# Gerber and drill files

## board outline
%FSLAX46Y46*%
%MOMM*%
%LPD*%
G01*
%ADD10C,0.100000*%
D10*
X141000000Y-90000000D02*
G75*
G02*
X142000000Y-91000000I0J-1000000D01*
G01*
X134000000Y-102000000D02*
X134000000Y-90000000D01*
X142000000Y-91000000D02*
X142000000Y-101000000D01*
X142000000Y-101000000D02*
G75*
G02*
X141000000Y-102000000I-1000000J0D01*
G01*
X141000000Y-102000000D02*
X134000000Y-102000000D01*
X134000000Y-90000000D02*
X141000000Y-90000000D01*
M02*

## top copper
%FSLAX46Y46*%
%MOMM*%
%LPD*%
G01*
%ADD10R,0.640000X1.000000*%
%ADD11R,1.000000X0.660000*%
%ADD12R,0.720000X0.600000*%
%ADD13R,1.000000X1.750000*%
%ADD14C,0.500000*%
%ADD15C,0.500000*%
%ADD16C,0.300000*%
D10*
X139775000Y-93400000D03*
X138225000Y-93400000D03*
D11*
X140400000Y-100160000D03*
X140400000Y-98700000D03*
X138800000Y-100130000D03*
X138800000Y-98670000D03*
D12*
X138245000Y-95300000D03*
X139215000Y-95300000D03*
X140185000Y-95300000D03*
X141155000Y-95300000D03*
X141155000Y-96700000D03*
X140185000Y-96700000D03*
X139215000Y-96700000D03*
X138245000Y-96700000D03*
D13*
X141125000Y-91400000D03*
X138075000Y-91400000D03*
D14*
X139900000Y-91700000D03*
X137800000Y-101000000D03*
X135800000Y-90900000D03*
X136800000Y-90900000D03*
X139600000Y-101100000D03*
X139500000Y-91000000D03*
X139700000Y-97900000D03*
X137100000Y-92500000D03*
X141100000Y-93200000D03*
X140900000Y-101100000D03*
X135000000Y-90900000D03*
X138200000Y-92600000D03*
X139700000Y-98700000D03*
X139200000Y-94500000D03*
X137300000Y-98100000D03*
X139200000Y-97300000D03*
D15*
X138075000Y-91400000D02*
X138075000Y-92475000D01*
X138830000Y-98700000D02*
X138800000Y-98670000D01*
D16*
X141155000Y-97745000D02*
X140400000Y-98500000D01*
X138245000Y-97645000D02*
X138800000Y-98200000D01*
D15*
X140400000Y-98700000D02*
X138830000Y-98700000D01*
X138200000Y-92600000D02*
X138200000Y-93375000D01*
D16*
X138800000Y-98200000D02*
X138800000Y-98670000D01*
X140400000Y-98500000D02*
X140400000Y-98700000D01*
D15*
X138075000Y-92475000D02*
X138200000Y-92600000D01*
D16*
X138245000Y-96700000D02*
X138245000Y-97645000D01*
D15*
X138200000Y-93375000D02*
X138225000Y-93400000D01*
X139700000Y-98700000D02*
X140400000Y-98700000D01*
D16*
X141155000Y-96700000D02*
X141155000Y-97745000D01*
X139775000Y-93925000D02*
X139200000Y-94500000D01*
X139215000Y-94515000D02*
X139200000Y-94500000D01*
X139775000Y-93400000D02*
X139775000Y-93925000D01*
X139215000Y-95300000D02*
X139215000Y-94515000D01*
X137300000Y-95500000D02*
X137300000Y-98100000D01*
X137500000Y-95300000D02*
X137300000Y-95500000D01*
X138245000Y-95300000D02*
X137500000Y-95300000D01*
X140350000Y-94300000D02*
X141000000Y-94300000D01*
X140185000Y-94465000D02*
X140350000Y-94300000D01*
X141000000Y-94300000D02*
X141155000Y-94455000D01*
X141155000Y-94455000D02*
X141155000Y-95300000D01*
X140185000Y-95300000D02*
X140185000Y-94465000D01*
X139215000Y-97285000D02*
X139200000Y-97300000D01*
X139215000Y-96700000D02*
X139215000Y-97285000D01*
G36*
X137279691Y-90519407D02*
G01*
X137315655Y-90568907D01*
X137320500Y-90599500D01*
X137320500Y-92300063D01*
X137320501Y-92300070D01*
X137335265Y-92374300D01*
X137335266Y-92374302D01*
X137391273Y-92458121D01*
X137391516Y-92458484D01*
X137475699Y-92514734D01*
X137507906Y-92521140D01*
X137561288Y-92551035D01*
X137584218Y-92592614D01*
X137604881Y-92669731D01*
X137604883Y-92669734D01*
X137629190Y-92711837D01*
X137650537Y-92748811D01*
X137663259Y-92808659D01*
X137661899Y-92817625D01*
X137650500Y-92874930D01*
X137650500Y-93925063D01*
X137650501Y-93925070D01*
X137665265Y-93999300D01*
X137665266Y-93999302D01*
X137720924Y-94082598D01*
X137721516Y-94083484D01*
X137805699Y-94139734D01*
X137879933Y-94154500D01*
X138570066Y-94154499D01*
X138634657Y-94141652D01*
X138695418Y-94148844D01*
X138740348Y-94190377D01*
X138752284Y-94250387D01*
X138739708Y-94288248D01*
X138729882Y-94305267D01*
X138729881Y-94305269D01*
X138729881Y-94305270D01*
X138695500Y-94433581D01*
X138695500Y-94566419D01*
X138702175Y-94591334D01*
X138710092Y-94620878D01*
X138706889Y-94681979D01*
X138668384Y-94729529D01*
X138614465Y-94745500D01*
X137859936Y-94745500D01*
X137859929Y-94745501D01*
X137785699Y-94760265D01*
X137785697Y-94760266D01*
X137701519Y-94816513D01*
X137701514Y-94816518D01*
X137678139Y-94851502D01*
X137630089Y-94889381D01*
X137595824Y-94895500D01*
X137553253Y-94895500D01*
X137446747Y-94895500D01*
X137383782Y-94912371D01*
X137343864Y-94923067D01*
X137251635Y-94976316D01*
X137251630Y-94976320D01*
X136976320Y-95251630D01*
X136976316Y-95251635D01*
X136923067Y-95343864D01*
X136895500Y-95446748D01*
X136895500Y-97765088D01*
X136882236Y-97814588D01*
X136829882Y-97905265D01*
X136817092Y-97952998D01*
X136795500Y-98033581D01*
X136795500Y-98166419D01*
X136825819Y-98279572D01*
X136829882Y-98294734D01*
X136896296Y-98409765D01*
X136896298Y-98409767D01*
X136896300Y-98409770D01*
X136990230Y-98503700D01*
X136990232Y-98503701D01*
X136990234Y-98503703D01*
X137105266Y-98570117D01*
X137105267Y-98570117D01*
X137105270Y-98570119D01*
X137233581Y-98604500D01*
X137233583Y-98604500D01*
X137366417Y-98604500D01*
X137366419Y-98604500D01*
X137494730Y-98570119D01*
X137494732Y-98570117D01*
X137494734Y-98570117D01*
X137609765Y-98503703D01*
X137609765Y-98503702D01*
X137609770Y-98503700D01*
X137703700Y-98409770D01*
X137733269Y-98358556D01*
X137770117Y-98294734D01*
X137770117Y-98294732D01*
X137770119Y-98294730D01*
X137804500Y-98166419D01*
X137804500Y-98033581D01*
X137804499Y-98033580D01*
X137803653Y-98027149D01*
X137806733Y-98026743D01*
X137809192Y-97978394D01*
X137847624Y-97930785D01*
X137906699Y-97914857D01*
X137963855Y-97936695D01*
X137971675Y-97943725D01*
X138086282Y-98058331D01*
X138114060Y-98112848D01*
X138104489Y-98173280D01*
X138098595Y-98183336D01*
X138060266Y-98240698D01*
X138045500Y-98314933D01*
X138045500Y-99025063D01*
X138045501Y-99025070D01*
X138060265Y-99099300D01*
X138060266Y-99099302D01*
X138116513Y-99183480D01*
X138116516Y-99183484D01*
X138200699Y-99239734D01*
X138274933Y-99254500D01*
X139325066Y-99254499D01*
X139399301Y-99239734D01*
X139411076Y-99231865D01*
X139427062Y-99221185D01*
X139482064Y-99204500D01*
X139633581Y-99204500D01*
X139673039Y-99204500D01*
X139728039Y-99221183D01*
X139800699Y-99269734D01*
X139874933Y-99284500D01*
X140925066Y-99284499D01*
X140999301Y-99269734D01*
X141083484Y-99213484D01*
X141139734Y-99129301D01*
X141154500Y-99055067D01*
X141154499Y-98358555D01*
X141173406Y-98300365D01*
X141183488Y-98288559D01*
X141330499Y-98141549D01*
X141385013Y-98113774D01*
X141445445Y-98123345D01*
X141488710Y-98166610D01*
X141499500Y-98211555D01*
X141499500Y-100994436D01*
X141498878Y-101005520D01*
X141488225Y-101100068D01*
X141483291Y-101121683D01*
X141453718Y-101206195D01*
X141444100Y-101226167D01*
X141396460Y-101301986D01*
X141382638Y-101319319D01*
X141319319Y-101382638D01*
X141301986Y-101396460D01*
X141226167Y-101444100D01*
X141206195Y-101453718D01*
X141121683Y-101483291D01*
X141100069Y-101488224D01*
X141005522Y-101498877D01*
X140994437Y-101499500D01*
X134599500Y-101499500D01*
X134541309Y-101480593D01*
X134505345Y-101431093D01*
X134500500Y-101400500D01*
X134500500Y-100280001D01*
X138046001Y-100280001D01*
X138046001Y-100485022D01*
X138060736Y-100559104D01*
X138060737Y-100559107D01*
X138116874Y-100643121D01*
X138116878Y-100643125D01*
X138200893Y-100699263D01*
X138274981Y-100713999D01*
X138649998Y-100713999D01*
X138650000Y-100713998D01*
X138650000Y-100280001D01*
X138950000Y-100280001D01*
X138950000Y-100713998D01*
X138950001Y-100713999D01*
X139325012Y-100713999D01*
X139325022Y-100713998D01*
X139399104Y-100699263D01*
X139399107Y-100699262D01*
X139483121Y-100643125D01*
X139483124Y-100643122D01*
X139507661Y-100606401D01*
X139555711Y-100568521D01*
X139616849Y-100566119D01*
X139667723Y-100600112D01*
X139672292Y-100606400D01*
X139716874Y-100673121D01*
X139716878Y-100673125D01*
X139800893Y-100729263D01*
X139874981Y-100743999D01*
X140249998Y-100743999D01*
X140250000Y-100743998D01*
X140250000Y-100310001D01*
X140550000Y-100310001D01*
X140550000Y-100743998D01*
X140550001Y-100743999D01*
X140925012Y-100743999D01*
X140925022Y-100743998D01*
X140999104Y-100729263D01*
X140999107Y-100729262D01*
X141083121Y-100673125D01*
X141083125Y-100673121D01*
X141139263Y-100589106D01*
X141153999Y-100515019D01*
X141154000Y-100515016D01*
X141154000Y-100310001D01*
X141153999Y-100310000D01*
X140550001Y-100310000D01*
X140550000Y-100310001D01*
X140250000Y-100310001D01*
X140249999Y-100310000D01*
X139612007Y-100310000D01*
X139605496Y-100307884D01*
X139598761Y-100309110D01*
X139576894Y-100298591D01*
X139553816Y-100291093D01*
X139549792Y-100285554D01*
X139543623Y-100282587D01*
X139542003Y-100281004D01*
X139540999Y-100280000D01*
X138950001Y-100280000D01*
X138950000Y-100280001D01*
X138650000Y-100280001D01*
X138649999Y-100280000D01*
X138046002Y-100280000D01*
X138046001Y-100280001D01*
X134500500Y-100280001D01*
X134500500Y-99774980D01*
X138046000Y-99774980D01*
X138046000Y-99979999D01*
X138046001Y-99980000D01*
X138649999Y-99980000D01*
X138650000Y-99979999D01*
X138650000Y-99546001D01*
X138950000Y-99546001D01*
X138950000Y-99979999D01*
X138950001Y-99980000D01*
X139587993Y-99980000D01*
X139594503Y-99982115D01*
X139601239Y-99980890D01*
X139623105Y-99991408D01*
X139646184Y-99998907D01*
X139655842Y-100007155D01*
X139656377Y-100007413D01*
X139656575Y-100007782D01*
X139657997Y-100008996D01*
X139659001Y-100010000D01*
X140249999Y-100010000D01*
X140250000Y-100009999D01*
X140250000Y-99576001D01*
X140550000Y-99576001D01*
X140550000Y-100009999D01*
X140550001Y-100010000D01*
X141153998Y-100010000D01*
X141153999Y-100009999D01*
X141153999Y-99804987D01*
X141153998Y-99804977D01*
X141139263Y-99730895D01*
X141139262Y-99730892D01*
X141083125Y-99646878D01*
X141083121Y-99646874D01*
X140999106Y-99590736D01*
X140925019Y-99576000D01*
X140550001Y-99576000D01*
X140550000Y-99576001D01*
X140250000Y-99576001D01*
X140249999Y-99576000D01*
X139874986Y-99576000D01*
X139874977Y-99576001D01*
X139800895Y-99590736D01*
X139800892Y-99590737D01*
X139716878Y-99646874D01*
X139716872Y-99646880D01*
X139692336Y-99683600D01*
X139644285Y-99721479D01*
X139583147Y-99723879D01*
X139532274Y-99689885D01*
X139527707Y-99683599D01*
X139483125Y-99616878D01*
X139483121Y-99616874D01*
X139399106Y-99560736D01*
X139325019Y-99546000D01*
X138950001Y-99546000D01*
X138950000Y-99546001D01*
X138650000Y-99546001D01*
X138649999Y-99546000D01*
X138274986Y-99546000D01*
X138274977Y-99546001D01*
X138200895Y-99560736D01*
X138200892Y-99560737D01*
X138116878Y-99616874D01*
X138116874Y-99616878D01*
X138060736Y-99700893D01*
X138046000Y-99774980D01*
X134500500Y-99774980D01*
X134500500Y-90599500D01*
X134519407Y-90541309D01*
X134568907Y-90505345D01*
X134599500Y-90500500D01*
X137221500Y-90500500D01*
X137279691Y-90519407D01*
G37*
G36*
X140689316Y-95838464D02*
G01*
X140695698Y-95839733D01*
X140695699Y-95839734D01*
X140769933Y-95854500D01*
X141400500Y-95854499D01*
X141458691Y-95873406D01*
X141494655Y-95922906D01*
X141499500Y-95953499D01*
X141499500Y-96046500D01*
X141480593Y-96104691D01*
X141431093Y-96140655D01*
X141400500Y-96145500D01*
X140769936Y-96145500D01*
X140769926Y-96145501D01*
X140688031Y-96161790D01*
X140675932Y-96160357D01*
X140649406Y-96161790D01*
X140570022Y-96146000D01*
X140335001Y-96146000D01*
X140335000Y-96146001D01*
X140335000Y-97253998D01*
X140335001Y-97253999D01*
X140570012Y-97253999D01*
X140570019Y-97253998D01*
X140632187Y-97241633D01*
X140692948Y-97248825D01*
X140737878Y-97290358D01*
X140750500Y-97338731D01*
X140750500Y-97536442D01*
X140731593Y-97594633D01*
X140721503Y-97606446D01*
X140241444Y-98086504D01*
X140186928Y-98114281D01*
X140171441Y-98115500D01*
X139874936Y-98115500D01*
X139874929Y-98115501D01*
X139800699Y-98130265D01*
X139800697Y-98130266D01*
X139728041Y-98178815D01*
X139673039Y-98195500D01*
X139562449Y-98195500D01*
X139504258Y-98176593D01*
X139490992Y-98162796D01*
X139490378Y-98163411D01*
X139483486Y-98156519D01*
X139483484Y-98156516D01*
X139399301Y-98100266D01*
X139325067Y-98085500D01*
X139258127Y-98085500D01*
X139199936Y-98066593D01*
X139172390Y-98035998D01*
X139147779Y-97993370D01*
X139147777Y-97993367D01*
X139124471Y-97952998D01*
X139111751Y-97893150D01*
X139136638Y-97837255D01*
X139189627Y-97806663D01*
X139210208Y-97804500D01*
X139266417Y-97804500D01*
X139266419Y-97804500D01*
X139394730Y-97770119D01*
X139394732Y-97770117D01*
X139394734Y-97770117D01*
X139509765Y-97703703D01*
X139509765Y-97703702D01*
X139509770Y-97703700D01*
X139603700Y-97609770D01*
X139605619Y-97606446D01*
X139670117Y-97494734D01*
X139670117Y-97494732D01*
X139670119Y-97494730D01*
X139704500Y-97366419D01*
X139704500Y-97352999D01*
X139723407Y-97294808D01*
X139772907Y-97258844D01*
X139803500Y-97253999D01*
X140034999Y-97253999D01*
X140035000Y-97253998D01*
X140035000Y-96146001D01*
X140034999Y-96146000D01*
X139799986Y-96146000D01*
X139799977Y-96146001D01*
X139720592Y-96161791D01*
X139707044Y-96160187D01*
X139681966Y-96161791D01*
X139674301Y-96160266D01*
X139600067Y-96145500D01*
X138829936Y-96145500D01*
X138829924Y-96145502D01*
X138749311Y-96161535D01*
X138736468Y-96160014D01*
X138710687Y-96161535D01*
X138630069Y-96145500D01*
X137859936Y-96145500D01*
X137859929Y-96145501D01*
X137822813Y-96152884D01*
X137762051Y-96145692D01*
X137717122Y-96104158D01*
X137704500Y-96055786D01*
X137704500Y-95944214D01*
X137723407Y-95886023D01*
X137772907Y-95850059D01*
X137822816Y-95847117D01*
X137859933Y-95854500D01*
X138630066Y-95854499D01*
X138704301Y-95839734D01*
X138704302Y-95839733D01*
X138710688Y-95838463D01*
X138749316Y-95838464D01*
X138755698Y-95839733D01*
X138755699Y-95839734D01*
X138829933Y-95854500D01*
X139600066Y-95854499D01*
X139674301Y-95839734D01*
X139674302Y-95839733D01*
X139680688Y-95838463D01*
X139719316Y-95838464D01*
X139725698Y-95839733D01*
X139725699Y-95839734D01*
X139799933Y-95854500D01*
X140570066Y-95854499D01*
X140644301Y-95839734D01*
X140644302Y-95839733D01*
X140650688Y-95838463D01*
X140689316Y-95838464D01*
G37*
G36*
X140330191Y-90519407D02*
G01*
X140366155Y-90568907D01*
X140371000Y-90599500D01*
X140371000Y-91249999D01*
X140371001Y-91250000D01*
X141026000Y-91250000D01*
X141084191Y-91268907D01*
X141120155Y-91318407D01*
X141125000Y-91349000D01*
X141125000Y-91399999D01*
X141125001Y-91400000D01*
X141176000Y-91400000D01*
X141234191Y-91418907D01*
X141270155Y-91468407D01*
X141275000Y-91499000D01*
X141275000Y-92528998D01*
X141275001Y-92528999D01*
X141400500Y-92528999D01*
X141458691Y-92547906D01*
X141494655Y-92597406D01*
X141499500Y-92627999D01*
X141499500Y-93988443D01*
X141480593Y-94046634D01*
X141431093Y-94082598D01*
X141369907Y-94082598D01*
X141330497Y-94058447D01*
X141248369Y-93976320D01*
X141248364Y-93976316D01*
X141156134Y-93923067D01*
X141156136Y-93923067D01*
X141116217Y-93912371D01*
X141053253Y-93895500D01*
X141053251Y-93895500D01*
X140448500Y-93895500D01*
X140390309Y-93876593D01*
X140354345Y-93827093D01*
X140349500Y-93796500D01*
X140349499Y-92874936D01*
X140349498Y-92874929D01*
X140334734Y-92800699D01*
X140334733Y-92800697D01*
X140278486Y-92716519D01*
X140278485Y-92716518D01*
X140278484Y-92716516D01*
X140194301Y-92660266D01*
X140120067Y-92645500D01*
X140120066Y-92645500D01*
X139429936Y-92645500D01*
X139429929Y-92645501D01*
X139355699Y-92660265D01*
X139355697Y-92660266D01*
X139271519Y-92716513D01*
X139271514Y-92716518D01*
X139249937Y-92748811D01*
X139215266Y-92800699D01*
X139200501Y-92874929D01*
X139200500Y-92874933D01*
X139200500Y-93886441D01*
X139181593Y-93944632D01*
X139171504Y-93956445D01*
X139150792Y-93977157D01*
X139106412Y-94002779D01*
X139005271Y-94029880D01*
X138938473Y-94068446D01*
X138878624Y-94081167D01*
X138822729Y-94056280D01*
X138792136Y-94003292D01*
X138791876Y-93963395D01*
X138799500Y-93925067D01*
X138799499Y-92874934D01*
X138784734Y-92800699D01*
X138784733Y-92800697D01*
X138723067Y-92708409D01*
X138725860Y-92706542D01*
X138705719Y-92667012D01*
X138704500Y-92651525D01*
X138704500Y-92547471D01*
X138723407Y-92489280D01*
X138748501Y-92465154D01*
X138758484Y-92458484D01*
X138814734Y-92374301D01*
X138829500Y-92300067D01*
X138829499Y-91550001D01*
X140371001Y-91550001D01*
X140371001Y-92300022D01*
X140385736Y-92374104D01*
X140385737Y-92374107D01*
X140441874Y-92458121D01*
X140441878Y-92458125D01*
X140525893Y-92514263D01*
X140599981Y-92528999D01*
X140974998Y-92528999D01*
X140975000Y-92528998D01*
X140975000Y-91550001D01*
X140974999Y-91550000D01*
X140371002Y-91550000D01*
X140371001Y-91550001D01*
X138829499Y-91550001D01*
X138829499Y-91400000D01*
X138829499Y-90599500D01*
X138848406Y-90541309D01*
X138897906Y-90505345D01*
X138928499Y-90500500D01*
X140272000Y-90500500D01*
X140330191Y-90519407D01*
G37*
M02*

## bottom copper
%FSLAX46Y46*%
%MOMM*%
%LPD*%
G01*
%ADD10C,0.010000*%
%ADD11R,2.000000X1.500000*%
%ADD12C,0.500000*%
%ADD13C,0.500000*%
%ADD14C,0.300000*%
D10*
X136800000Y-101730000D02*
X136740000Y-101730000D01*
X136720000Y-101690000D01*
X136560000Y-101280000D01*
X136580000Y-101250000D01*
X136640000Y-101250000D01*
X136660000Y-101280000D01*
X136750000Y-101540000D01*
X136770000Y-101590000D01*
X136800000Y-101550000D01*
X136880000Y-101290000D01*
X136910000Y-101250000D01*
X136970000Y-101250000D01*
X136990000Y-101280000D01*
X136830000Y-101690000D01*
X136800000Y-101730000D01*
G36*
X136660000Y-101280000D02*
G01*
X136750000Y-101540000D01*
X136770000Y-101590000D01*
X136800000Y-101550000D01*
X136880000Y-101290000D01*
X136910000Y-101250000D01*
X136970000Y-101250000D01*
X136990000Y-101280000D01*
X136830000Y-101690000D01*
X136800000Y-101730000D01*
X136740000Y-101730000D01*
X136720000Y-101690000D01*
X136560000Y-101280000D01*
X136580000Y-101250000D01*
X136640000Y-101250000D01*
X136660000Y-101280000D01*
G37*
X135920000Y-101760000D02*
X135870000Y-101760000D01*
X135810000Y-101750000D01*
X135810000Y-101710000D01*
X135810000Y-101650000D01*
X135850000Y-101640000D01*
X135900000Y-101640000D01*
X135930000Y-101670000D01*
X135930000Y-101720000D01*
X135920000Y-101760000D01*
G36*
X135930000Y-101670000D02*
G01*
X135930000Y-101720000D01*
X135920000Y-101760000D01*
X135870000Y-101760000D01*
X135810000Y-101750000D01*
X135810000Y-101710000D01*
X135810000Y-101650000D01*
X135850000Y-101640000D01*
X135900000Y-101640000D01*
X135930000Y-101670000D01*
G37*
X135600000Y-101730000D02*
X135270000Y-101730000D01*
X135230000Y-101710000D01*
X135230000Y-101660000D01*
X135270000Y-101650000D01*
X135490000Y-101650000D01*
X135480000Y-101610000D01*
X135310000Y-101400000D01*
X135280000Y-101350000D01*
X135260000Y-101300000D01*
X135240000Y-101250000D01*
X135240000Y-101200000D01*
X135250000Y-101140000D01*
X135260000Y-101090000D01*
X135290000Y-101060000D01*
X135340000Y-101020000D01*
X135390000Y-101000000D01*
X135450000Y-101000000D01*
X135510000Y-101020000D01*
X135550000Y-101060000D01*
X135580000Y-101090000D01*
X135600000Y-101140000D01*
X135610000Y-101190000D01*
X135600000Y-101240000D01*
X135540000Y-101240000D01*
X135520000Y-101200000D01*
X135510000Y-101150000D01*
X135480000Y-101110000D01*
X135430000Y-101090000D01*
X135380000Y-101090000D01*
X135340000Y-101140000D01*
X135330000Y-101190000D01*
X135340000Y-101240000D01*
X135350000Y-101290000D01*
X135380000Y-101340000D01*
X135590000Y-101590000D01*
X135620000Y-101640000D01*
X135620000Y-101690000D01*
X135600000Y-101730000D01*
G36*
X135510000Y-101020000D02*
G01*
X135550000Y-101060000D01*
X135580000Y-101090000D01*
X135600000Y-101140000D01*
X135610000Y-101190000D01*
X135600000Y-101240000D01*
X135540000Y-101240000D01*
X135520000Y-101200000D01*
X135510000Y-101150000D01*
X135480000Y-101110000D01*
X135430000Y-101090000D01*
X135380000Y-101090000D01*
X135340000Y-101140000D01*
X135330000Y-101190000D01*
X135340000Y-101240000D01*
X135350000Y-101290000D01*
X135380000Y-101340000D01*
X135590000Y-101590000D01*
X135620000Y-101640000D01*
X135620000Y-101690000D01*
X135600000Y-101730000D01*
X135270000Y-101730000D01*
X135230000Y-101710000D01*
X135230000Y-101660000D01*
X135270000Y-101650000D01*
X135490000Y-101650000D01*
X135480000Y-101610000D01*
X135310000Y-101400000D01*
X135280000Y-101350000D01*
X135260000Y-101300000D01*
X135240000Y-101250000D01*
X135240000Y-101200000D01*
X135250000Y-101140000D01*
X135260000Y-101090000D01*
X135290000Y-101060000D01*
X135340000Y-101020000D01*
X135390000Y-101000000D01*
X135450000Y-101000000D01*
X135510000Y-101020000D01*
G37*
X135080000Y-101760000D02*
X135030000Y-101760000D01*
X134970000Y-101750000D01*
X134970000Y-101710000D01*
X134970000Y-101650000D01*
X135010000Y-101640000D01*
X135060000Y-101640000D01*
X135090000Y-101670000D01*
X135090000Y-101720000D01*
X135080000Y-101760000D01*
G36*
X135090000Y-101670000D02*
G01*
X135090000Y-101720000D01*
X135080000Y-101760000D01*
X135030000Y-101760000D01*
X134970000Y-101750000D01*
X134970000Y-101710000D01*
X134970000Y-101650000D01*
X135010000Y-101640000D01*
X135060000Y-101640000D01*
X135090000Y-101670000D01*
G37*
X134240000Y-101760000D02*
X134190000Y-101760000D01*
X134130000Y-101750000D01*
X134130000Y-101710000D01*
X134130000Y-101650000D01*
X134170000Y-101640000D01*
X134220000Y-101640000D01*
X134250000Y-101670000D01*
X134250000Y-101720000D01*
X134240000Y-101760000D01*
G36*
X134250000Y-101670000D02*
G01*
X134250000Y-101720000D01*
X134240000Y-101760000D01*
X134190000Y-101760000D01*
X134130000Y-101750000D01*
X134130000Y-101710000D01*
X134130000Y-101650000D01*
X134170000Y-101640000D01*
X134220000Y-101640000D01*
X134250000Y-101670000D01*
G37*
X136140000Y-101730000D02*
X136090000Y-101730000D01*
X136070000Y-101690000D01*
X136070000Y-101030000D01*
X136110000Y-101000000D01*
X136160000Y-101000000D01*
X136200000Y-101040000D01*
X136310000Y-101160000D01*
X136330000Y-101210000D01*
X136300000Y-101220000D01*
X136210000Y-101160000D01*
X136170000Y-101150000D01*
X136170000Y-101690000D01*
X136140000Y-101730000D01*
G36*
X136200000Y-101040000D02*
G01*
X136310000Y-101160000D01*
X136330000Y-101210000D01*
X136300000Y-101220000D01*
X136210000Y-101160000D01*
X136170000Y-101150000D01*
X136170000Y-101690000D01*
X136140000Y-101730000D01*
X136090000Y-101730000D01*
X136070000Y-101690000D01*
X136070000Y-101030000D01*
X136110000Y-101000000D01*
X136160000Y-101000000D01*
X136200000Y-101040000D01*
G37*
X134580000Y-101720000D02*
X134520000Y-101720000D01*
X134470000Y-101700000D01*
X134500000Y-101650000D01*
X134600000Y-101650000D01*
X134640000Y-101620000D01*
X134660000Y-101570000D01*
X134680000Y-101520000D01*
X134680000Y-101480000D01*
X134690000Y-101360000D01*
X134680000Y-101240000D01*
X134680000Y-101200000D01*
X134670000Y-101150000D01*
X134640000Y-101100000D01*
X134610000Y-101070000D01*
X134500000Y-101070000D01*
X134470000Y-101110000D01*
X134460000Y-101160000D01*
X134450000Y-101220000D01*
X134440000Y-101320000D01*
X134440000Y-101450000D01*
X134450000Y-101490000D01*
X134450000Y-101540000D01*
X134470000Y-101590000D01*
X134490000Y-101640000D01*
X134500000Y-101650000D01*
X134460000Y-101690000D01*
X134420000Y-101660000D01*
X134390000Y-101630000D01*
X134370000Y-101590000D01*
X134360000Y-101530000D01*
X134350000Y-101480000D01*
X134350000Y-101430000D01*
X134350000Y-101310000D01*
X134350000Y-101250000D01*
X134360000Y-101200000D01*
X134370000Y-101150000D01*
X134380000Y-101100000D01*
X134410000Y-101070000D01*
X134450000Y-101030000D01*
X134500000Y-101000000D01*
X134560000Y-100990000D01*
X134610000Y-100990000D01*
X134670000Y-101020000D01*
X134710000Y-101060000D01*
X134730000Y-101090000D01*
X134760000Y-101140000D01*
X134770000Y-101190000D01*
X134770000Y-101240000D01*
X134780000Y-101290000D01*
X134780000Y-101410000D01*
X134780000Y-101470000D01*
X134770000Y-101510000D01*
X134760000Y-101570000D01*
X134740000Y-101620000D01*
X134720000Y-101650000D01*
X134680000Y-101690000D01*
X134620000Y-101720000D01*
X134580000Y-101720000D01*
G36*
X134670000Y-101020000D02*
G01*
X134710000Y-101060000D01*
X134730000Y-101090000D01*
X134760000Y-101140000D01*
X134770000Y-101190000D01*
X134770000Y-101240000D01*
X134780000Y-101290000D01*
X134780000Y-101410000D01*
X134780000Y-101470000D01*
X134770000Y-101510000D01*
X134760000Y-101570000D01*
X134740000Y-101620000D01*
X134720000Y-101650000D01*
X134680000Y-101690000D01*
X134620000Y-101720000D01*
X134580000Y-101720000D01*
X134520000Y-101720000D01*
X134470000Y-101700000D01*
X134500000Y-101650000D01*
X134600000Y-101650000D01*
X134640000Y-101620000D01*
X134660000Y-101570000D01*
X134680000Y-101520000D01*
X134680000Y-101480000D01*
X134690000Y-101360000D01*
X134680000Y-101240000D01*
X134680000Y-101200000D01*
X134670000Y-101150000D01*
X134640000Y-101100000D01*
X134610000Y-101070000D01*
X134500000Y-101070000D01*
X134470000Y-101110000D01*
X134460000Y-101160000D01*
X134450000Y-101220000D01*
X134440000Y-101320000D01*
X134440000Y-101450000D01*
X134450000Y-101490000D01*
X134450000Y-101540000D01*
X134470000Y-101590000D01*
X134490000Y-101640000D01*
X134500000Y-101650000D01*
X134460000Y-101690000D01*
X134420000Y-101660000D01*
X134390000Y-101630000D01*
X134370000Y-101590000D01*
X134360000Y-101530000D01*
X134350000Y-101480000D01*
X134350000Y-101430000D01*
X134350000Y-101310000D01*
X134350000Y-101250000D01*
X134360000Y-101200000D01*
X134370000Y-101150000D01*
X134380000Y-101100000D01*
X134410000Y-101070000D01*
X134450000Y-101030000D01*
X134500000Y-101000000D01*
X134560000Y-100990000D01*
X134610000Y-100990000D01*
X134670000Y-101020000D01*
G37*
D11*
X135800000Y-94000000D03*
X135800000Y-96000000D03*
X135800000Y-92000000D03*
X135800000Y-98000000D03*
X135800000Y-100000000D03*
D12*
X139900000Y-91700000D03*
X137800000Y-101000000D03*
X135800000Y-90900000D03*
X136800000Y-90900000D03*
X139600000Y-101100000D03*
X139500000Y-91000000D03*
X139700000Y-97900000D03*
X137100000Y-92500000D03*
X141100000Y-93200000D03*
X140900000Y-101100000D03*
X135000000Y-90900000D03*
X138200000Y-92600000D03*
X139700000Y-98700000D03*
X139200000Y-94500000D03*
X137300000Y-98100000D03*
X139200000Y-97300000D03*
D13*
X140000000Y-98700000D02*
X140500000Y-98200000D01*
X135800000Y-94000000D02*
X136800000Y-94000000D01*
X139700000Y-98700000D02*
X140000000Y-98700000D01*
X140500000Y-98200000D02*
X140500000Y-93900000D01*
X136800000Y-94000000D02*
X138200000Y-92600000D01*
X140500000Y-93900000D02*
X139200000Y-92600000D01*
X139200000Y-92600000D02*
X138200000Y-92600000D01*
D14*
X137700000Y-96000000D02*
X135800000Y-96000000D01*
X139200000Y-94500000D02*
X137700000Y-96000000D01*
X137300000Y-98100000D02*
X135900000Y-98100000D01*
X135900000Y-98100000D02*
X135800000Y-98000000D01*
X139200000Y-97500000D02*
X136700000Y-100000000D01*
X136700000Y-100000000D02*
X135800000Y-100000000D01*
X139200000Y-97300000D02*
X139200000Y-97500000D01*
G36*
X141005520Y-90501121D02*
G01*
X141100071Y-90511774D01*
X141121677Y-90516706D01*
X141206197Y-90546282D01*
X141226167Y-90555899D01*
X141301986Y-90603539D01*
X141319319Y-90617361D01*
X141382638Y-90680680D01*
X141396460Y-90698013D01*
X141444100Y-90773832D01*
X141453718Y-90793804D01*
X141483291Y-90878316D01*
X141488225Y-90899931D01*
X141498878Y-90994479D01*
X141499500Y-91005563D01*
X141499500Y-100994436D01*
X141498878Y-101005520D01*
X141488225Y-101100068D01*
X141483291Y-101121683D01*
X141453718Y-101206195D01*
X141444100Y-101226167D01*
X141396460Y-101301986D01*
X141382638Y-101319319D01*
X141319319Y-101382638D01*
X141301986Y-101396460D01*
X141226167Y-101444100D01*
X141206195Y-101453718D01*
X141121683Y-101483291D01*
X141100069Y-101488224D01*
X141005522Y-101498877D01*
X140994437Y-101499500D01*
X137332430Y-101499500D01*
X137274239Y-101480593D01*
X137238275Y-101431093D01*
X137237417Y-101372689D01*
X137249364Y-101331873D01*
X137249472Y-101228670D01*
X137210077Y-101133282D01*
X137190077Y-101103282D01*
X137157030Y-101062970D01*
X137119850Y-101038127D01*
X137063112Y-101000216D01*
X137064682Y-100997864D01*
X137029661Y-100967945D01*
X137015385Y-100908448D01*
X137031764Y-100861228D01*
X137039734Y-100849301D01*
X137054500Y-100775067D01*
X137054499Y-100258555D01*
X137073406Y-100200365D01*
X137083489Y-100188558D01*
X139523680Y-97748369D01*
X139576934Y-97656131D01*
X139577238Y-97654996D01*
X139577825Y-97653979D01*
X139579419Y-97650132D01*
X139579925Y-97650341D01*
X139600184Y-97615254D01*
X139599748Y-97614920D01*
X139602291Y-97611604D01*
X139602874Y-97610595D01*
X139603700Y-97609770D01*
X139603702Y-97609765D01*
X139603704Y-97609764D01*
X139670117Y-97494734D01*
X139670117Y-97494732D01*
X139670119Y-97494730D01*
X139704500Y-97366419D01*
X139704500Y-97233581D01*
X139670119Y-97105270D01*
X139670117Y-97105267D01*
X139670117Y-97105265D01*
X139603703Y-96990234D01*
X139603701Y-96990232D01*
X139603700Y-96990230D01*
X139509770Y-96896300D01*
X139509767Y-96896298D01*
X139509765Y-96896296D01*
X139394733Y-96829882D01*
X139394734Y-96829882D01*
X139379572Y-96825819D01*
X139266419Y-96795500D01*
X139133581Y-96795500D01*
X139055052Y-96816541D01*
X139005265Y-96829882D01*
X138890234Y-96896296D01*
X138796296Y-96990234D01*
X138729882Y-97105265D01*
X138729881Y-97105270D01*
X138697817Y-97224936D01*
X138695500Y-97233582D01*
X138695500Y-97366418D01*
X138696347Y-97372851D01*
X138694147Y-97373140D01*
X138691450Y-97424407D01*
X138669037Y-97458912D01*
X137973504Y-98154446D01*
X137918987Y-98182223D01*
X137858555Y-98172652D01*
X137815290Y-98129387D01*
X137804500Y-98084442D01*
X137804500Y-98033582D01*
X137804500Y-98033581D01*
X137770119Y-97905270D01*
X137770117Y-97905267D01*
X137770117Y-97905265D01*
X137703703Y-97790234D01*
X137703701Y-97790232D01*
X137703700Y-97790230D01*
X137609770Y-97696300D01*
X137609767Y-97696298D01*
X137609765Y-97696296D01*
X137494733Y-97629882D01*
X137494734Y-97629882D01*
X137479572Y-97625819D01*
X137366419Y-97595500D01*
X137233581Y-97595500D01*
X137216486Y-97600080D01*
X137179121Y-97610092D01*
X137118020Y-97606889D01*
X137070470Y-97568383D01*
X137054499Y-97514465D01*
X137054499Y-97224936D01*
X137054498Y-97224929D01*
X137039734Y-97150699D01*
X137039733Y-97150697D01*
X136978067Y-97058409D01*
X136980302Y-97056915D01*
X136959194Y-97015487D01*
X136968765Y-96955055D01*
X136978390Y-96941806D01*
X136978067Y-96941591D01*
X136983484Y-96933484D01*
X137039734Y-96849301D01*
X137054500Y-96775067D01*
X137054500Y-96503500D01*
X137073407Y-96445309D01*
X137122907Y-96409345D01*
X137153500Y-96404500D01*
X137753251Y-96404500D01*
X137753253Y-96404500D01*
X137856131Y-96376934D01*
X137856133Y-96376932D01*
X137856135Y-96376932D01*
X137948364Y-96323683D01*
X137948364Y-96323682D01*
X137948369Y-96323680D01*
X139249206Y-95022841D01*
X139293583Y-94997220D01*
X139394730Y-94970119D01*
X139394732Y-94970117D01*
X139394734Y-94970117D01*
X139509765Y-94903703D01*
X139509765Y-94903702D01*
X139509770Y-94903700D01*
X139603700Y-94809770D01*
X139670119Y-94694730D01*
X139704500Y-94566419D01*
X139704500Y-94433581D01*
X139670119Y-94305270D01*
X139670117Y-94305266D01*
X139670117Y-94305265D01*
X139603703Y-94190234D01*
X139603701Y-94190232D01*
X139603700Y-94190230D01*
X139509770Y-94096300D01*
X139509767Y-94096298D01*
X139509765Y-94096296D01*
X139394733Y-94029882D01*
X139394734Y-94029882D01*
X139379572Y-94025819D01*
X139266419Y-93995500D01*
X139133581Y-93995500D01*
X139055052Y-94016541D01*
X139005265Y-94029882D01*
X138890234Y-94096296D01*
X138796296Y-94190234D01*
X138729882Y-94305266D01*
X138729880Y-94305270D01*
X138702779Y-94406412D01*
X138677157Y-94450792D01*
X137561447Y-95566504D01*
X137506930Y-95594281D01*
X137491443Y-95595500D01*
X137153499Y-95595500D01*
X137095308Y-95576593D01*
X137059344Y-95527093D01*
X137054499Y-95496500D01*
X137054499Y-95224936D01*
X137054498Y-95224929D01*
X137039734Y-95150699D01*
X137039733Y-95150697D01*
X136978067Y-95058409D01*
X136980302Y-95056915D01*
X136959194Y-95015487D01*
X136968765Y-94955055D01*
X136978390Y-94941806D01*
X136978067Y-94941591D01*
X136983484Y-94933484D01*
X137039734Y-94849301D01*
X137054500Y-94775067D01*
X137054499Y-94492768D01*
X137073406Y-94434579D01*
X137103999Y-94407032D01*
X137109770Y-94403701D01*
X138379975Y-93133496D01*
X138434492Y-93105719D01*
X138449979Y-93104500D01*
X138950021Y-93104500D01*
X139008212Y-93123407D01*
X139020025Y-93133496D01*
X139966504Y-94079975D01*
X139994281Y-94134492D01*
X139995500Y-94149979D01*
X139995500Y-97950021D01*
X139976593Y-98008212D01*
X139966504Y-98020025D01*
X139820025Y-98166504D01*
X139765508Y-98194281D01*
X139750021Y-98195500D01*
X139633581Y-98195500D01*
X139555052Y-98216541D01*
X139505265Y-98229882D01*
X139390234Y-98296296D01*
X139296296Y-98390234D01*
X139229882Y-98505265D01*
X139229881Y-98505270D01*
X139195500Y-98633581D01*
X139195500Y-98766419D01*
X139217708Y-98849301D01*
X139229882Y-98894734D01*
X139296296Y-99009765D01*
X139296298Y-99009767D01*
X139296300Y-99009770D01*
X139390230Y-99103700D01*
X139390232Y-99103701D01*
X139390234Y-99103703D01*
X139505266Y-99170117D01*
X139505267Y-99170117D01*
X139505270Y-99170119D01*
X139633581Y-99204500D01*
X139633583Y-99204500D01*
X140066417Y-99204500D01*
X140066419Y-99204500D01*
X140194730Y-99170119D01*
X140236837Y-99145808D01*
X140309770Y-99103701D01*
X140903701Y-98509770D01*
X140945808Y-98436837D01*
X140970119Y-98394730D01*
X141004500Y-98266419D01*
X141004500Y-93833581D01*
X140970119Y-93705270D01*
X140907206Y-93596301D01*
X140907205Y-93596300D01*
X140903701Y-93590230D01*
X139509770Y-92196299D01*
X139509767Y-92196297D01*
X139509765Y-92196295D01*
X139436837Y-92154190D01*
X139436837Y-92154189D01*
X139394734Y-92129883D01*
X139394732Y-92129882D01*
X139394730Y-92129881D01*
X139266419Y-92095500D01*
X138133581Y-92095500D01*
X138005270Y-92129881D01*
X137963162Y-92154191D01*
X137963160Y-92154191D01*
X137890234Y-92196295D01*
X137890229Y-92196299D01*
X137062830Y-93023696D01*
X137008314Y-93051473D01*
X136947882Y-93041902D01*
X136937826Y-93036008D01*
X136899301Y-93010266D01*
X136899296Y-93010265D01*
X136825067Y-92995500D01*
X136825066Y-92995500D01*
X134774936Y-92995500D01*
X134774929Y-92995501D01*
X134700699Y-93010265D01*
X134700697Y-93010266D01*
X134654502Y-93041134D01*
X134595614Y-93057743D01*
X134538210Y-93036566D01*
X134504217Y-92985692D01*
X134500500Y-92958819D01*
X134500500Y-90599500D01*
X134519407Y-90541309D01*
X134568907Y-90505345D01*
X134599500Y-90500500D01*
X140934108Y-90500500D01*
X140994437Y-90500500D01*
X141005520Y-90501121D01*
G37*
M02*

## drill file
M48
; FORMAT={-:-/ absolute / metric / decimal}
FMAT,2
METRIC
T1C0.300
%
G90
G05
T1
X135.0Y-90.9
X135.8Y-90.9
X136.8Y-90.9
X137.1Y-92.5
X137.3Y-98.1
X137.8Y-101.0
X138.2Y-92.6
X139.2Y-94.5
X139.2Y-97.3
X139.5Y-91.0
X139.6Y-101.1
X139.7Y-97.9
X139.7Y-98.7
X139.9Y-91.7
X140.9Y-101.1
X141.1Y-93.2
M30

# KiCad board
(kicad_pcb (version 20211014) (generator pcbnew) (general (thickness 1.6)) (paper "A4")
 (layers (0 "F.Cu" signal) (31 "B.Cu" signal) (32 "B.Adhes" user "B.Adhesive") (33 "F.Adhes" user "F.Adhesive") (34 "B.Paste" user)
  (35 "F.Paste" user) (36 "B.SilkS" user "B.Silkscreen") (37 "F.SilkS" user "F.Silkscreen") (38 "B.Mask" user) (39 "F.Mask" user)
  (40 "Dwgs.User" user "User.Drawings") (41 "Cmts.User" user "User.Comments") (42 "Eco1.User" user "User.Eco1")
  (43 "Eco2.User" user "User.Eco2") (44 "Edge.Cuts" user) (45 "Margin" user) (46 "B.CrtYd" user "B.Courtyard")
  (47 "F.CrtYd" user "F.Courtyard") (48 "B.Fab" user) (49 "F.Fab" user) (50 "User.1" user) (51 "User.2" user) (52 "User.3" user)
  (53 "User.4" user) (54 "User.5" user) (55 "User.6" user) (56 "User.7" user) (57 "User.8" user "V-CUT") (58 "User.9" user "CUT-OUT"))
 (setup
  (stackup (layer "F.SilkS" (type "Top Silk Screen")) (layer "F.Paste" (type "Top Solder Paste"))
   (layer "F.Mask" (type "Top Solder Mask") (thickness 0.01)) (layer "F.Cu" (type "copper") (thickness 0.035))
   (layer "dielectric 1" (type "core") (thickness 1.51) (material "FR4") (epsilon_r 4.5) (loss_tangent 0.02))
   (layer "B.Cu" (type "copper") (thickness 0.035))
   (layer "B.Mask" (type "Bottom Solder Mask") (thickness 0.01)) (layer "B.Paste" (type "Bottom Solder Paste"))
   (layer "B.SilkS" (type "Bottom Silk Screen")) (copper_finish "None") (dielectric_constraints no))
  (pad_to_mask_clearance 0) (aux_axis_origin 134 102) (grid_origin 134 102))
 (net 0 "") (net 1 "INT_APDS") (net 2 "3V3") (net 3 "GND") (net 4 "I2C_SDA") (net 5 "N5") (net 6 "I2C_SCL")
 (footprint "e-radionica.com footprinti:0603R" (layer "F.Cu") (at 139 93.4 180)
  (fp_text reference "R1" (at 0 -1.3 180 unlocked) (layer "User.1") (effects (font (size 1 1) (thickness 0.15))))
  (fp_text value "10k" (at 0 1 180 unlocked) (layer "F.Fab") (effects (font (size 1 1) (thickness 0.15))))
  (pad "1" smd rect locked (at -0.775 0 270) (size 1 0.64) (layers "F.Cu" "F.Paste" "F.Mask") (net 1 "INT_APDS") (solder_mask_margin 0.1))
  (pad "2" smd rect locked (at 0.775 0 270) (size 1 0.64) (layers "F.Cu" "F.Paste" "F.Mask") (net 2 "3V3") (solder_mask_margin 0.1)))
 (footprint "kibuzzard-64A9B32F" (layer "F.Cu") (at 135 96 -90)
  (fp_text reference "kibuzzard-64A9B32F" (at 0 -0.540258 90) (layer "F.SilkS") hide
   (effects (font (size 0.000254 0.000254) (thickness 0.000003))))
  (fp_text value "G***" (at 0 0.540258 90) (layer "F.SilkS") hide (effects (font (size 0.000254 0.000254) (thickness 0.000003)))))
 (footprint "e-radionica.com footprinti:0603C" (layer "F.Cu") (at 140.4 99.43 90)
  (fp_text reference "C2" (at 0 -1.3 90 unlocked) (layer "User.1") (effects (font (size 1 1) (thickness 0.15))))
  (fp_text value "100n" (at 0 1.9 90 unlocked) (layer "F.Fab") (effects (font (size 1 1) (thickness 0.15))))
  (pad "1" smd rect locked (at -0.73 0 90) (size 0.66 1) (layers "F.Cu" "F.Paste" "F.Mask") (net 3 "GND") (solder_mask_margin 0.1))
  (pad "2" smd rect locked (at 0.73 0 90) (size 0.66 1) (layers "F.Cu" "F.Paste" "F.Mask") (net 2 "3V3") (solder_mask_margin 0.1)))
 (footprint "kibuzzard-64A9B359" (layer "F.Cu") (at 136.5 96 -90)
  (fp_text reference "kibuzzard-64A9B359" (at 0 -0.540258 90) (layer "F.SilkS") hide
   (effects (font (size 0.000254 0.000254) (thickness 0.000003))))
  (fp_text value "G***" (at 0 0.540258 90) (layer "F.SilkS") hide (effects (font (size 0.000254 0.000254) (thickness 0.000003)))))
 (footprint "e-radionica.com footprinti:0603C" (layer "F.Cu") (at 138.8 99.4 90)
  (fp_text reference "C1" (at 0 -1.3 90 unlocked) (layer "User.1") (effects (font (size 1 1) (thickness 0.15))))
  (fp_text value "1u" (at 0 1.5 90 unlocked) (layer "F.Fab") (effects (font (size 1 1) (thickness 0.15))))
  (pad "1" smd rect locked (at -0.73 0 90) (size 0.66 1) (layers "F.Cu" "F.Paste" "F.Mask") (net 3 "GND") (solder_mask_margin 0.1))
  (pad "2" smd rect locked (at 0.73 0 90) (size 0.66 1) (layers "F.Cu" "F.Paste" "F.Mask") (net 2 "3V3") (solder_mask_margin 0.1)))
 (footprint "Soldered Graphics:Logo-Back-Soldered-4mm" (layer "F.Cu") (at 139.5 96 90)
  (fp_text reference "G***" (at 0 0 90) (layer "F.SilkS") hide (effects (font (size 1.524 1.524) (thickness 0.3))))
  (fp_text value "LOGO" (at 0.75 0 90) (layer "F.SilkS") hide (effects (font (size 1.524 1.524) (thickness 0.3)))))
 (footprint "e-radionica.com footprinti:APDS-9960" (layer "F.Cu") (at 139.7 96 90)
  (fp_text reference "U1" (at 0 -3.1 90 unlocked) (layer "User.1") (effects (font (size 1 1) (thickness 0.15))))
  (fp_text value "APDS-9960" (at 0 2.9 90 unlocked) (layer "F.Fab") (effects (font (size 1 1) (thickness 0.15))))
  (pad "1" smd rect (at 0.7 -1.455 90) (size 0.6 0.72) (layers "F.Cu" "F.Paste" "F.Mask") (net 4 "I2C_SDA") (solder_mask_margin 0.1))
  (pad "2" smd rect (at 0.7 -0.485 90) (size 0.6 0.72) (layers "F.Cu" "F.Paste" "F.Mask") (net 1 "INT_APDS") (solder_mask_margin 0.1))
  (pad "3" smd rect (at 0.7 0.485 90) (size 0.6 0.72) (layers "F.Cu" "F.Paste" "F.Mask") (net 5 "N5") (solder_mask_margin 0.1))
  (pad "4" smd rect (at 0.7 1.455 90) (size 0.6 0.72) (layers "F.Cu" "F.Paste" "F.Mask") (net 5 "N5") (solder_mask_margin 0.1))
  (pad "5" smd rect (at -0.7 1.455 90) (size 0.6 0.72) (layers "F.Cu" "F.Paste" "F.Mask") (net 2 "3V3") (solder_mask_margin 0.1))
  (pad "6" smd rect (at -0.7 0.485 90) (size 0.6 0.72) (layers "F.Cu" "F.Paste" "F.Mask") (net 3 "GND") (solder_mask_margin 0.1))
  (pad "7" smd rect (at -0.7 -0.485 90) (size 0.6 0.72) (layers "F.Cu" "F.Paste" "F.Mask") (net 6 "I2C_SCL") (solder_mask_margin 0.1))
  (pad "8" smd rect (at -0.7 -1.455 90) (size 0.6 0.72) (layers "F.Cu" "F.Paste" "F.Mask") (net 2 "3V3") (solder_mask_margin 0.1)))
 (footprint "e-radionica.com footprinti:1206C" (layer "F.Cu") (at 139.6 91.4 180)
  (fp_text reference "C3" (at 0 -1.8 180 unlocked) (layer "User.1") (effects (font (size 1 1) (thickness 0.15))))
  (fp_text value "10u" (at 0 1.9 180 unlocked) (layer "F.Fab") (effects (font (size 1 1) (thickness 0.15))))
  (pad "1" smd rect locked (at -1.525 0 270) (size 1.75 1) (layers "F.Cu" "F.Paste" "F.Mask") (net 3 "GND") (solder_mask_margin 0.1))
  (pad "2" smd rect locked (at 1.525 0 270) (size 1.75 1) (layers "F.Cu" "F.Paste" "F.Mask") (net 2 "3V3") (solder_mask_margin 0.1)))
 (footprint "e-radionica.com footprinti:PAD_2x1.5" (layer "B.Cu") (at 135.8 94 180)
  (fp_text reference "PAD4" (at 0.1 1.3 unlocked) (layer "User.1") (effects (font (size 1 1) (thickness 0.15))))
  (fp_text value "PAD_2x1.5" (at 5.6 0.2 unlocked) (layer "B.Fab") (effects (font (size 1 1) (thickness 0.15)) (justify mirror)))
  (pad "1" smd rect (at 0 0 180) (size 2 1.5) (layers "B.Cu" "B.Paste" "B.Mask") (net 2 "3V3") (solder_mask_margin 0.1)))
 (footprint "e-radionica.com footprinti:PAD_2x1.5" (layer "B.Cu") (at 135.8 96 180)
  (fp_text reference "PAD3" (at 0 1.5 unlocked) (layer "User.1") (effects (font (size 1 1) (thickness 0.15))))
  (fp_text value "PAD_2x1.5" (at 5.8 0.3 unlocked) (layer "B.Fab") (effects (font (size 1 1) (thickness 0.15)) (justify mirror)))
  (pad "1" smd rect (at 0 0 180) (size 2 1.5) (layers "B.Cu" "B.Paste" "B.Mask") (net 1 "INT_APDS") (solder_mask_margin 0.1)))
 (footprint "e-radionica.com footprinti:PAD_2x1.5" (layer "B.Cu") (at 135.8 92 180)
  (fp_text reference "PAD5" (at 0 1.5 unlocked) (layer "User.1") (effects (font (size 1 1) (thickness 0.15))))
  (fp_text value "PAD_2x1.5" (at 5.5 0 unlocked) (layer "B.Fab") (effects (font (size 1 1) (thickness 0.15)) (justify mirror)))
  (pad "1" smd rect (at 0 0 180) (size 2 1.5) (layers "B.Cu" "B.Paste" "B.Mask") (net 3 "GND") (solder_mask_margin 0.1) (zone_connect 2)))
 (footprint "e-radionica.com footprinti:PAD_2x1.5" (layer "B.Cu") (at 135.8 98 180)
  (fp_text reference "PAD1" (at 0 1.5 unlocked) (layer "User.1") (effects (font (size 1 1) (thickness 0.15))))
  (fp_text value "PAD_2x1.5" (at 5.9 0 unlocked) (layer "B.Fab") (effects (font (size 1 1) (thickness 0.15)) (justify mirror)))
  (pad "1" smd rect (at 0 0 180) (size 2 1.5) (layers "B.Cu" "B.Paste" "B.Mask") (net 4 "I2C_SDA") (solder_mask_margin 0.1)))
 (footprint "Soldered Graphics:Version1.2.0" (layer "B.Cu") (at 135.5 101.4 180)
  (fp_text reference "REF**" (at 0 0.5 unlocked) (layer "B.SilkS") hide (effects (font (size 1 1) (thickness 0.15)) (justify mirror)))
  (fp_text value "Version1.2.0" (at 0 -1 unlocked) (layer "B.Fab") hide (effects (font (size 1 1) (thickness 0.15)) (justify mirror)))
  (fp_poly
   (pts (xy -1.3 -0.33) (xy -1.24 -0.33) (xy -1.22 -0.29) (xy -1.06 0.12) (xy -1.08 0.15) (xy -1.14 0.15) (xy -1.16 0.12) (xy -1.25 -0.14)
    (xy -1.27 -0.19) (xy -1.3 -0.15) (xy -1.38 0.11) (xy -1.41 0.15) (xy -1.47 0.15) (xy -1.49 0.12) (xy -1.33 -0.29) (xy -1.3 -0.33))
   (layer "B.Cu") (width 0.01) (fill solid))
  (fp_poly
   (pts (xy -0.42 -0.36) (xy -0.37 -0.36) (xy -0.31 -0.35) (xy -0.31 -0.31) (xy -0.31 -0.25) (xy -0.35 -0.24) (xy -0.4 -0.24)
    (xy -0.43 -0.27) (xy -0.43 -0.32) (xy -0.42 -0.36))
   (layer "B.Cu") (width 0.01) (fill solid))
  (fp_poly
   (pts (xy -0.1 -0.33) (xy 0.23 -0.33) (xy 0.27 -0.31) (xy 0.27 -0.26) (xy 0.23 -0.25) (xy 0.01 -0.25) (xy 0.02 -0.21) (xy 0.19 0)
    (xy 0.22 0.05) (xy 0.24 0.1) (xy 0.26 0.15) (xy 0.26 0.2) (xy 0.25 0.26) (xy 0.24 0.31) (xy 0.21 0.34) (xy 0.16 0.38) (xy 0.11 0.4)
    (xy 0.05 0.4) (xy -0.01 0.38) (xy -0.05 0.34) (xy -0.08 0.31) (xy -0.1 0.26) (xy -0.11 0.21) (xy -0.1 0.16) (xy -0.04 0.16)
    (xy -0.02 0.2) (xy -0.01 0.25) (xy 0.02 0.29) (xy 0.07 0.31) (xy 0.12 0.31) (xy 0.16 0.26) (xy 0.17 0.21) (xy 0.16 0.16) (xy 0.15 0.11)
    (xy 0.12 0.06) (xy -0.09 -0.19) (xy -0.12 -0.24) (xy -0.12 -0.29) (xy -0.1 -0.33))
   (layer "B.Cu") (width 0.01) (fill solid))
  (fp_poly
   (pts (xy 0.42 -0.36) (xy 0.47 -0.36) (xy 0.53 -0.35) (xy 0.53 -0.31) (xy 0.53 -0.25) (xy 0.49 -0.24) (xy 0.44 -0.24) (xy 0.41 -0.27)
    (xy 0.41 -0.32) (xy 0.42 -0.36))
   (layer "B.Cu") (width 0.01) (fill solid))
  (fp_poly
   (pts (xy 1.26 -0.36) (xy 1.31 -0.36) (xy 1.37 -0.35) (xy 1.37 -0.31) (xy 1.37 -0.25) (xy 1.33 -0.24) (xy 1.28 -0.24) (xy 1.25 -0.27)
    (xy 1.25 -0.32) (xy 1.26 -0.36))
   (layer "B.Cu") (width 0.01) (fill solid))
  (fp_poly
   (pts (xy -0.64 -0.33) (xy -0.59 -0.33) (xy -0.57 -0.29) (xy -0.57 0.37) (xy -0.61 0.4) (xy -0.66 0.4) (xy -0.7 0.36) (xy -0.81 0.24)
    (xy -0.83 0.19) (xy -0.8 0.18) (xy -0.71 0.24) (xy -0.67 0.25) (xy -0.67 -0.29) (xy -0.64 -0.33))
   (layer "B.Cu") (width 0.01) (fill solid))
  (fp_poly
   (pts (xy 0.92 -0.32) (xy 0.98 -0.32) (xy 1.03 -0.3) (xy 1 -0.25) (xy 0.9 -0.25) (xy 0.86 -0.22) (xy 0.84 -0.17) (xy 0.82 -0.12)
    (xy 0.82 -0.08) (xy 0.81 0.04) (xy 0.82 0.16) (xy 0.82 0.2) (xy 0.83 0.25) (xy 0.86 0.3) (xy 0.89 0.33) (xy 1 0.33) (xy 1.03 0.29)
    (xy 1.04 0.24) (xy 1.05 0.18) (xy 1.06 0.08) (xy 1.06 -0.05) (xy 1.05 -0.09) (xy 1.05 -0.14) (xy 1.03 -0.19) (xy 1.01 -0.24)
    (xy 1 -0.25) (xy 1.04 -0.29) (xy 1.08 -0.26) (xy 1.11 -0.23) (xy 1.13 -0.19) (xy 1.14 -0.13) (xy 1.15 -0.08) (xy 1.15 -0.03)
    (xy 1.15 0.09) (xy 1.15 0.15) (xy 1.14 0.2) (xy 1.13 0.25) (xy 1.12 0.3) (xy 1.09 0.33) (xy 1.05 0.37) (xy 1 0.4) (xy 0.94 0.41)
    (xy 0.89 0.41) (xy 0.83 0.38) (xy 0.79 0.34) (xy 0.77 0.31) (xy 0.74 0.26) (xy 0.73 0.21) (xy 0.73 0.16) (xy 0.72 0.11) (xy 0.72 -0.01)
    (xy 0.72 -0.07) (xy 0.73 -0.11) (xy 0.74 -0.17) (xy 0.76 -0.22) (xy 0.78 -0.25) (xy 0.82 -0.29) (xy 0.88 -0.32) (xy 0.92 -0.32))
   (layer "B.Cu") (width 0.01) (fill solid)))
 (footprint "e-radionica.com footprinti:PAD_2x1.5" (layer "B.Cu") (at 135.8 100 180)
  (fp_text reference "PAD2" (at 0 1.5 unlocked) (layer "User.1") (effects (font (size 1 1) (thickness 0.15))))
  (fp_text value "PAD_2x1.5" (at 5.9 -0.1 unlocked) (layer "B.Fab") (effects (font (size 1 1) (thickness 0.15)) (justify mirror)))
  (pad "1" smd rect (at 0 0 180) (size 2 1.5) (layers "B.Cu" "B.Paste" "B.Mask") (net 6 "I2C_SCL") (solder_mask_margin 0.1)))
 (gr_arc (start 141 90) (mid 141.707107 90.292893) (end 142 91) (layer "Edge.Cuts") (width 0.1))
 (gr_line (start 134 102) (end 134 90) (layer "Edge.Cuts") (width 0.1))
 (gr_line (start 142 91) (end 142 101) (layer "Edge.Cuts") (width 0.1))
 (gr_arc (start 142 101) (mid 141.707107 101.707107) (end 141 102) (layer "Edge.Cuts") (width 0.1))
 (gr_line (start 141 102) (end 134 102) (layer "Edge.Cuts") (width 0.1))
 (gr_line (start 134 90) (end 141 90) (layer "Edge.Cuts") (width 0.1))
 (via (at 139.9 91.7) (size 0.5) (drill 0.3) (layers "F.Cu" "B.Cu") (free) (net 3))
 (via (at 137.8 101) (size 0.5) (drill 0.3) (layers "F.Cu" "B.Cu") (free) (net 3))
 (via (at 135.8 90.9) (size 0.5) (drill 0.3) (layers "F.Cu" "B.Cu") (free) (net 3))
 (via (at 136.8 90.9) (size 0.5) (drill 0.3) (layers "F.Cu" "B.Cu") (free) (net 3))
 (via (at 139.6 101.1) (size 0.5) (drill 0.3) (layers "F.Cu" "B.Cu") (free) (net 3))
 (via (at 139.5 91) (size 0.5) (drill 0.3) (layers "F.Cu" "B.Cu") (free) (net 3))
 (via (at 139.7 97.9) (size 0.5) (drill 0.3) (layers "F.Cu" "B.Cu") (free) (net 3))
 (via (at 137.1 92.5) (size 0.5) (drill 0.3) (layers "F.Cu" "B.Cu") (free) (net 3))
 (via (at 141.1 93.2) (size 0.5) (drill 0.3) (layers "F.Cu" "B.Cu") (free) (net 3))
 (via (at 140.9 101.1) (size 0.5) (drill 0.3) (layers "F.Cu" "B.Cu") (free) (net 3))
 (via (at 135 90.9) (size 0.5) (drill 0.3) (layers "F.Cu" "B.Cu") (free) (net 3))
 (segment (start 138.075 91.4) (end 138.075 92.475) (width 0.5) (layer "F.Cu") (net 2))
 (segment (start 138.83 98.7) (end 138.8 98.67) (width 0.5) (layer "F.Cu") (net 2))
 (segment (start 141.155 97.745) (end 140.4 98.5) (width 0.3) (layer "F.Cu") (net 2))
 (segment (start 138.245 97.645) (end 138.8 98.2) (width 0.3) (layer "F.Cu") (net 2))
 (segment (start 140.4 98.7) (end 138.83 98.7) (width 0.5) (layer "F.Cu") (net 2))
 (segment (start 138.2 92.6) (end 138.2 93.375) (width 0.5) (layer "F.Cu") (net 2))
 (segment (start 138.8 98.2) (end 138.8 98.67) (width 0.3) (layer "F.Cu") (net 2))
 (segment (start 140.4 98.5) (end 140.4 98.7) (width 0.3) (layer "F.Cu") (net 2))
 (segment (start 138.075 92.475) (end 138.2 92.6) (width 0.5) (layer "F.Cu") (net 2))
 (segment (start 138.245 96.7) (end 138.245 97.645) (width 0.3) (layer "F.Cu") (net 2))
 (segment (start 138.2 93.375) (end 138.225 93.4) (width 0.5) (layer "F.Cu") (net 2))
 (segment (start 139.7 98.7) (end 140.4 98.7) (width 0.5) (layer "F.Cu") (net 2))
 (segment (start 141.155 96.7) (end 141.155 97.745) (width 0.3) (layer "F.Cu") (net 2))
 (via (at 138.2 92.6) (size 0.5) (drill 0.3) (layers "F.Cu" "B.Cu") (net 2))
 (via (at 139.7 98.7) (size 0.5) (drill 0.3) (layers "F.Cu" "B.Cu") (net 2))
 (segment (start 140 98.7) (end 140.5 98.2) (width 0.5) (layer "B.Cu") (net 2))
 (segment (start 135.8 94) (end 136.8 94) (width 0.5) (layer "B.Cu") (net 2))
 (segment (start 139.7 98.7) (end 140 98.7) (width 0.5) (layer "B.Cu") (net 2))
 (segment (start 140.5 98.2) (end 140.5 93.9) (width 0.5) (layer "B.Cu") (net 2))
 (segment (start 136.8 94) (end 138.2 92.6) (width 0.5) (layer "B.Cu") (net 2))
 (segment (start 140.5 93.9) (end 139.2 92.6) (width 0.5) (layer "B.Cu") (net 2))
 (segment (start 139.2 92.6) (end 138.2 92.6) (width 0.5) (layer "B.Cu") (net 2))
 (segment (start 139.775 93.925) (end 139.2 94.5) (width 0.3) (layer "F.Cu") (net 1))
 (segment (start 139.215 94.515) (end 139.2 94.5) (width 0.3) (layer "F.Cu") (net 1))
 (segment (start 139.775 93.4) (end 139.775 93.925) (width 0.3) (layer "F.Cu") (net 1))
 (segment (start 139.215 95.3) (end 139.215 94.515) (width 0.3) (layer "F.Cu") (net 1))
 (via (at 139.2 94.5) (size 0.5) (drill 0.3) (layers "F.Cu" "B.Cu") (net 1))
 (segment (start 137.7 96) (end 135.8 96) (width 0.3) (layer "B.Cu") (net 1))
 (segment (start 139.2 94.5) (end 137.7 96) (width 0.3) (layer "B.Cu") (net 1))
 (segment (start 137.3 95.5) (end 137.3 98.1) (width 0.3) (layer "F.Cu") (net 4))
 (segment (start 137.5 95.3) (end 137.3 95.5) (width 0.3) (layer "F.Cu") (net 4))
 (segment (start 138.245 95.3) (end 137.5 95.3) (width 0.3) (layer "F.Cu") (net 4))
 (via (at 137.3 98.1) (size 0.5) (drill 0.3) (layers "F.Cu" "B.Cu") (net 4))
 (segment (start 137.3 98.1) (end 135.9 98.1) (width 0.3) (layer "B.Cu") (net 4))
 (segment (start 135.9 98.1) (end 135.8 98) (width 0.3) (layer "B.Cu") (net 4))
 (segment (start 140.35 94.3) (end 141 94.3) (width 0.3) (layer "F.Cu") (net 5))
 (segment (start 140.185 94.465) (end 140.35 94.3) (width 0.3) (layer "F.Cu") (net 5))
 (segment (start 141 94.3) (end 141.155 94.455) (width 0.3) (layer "F.Cu") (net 5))
 (segment (start 141.155 94.455) (end 141.155 95.3) (width 0.3) (layer "F.Cu") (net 5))
 (segment (start 140.185 95.3) (end 140.185 94.465) (width 0.3) (layer "F.Cu") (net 5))
 (segment (start 139.215 97.285) (end 139.2 97.3) (width 0.3) (layer "F.Cu") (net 6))
 (segment (start 139.215 96.7) (end 139.215 97.285) (width 0.3) (layer "F.Cu") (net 6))
 (via (at 139.2 97.3) (size 0.5) (drill 0.3) (layers "F.Cu" "B.Cu") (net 6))
 (segment (start 139.2 97.5) (end 136.7 100) (width 0.3) (layer "B.Cu") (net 6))
 (segment (start 136.7 100) (end 135.8 100) (width 0.3) (layer "B.Cu") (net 6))
 (segment (start 139.2 97.3) (end 139.2 97.5) (width 0.3) (layer "B.Cu") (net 6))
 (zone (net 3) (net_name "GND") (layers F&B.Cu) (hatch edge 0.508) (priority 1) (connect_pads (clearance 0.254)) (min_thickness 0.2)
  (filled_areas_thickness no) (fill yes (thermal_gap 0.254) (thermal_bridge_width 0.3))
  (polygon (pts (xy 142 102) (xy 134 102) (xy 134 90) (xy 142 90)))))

